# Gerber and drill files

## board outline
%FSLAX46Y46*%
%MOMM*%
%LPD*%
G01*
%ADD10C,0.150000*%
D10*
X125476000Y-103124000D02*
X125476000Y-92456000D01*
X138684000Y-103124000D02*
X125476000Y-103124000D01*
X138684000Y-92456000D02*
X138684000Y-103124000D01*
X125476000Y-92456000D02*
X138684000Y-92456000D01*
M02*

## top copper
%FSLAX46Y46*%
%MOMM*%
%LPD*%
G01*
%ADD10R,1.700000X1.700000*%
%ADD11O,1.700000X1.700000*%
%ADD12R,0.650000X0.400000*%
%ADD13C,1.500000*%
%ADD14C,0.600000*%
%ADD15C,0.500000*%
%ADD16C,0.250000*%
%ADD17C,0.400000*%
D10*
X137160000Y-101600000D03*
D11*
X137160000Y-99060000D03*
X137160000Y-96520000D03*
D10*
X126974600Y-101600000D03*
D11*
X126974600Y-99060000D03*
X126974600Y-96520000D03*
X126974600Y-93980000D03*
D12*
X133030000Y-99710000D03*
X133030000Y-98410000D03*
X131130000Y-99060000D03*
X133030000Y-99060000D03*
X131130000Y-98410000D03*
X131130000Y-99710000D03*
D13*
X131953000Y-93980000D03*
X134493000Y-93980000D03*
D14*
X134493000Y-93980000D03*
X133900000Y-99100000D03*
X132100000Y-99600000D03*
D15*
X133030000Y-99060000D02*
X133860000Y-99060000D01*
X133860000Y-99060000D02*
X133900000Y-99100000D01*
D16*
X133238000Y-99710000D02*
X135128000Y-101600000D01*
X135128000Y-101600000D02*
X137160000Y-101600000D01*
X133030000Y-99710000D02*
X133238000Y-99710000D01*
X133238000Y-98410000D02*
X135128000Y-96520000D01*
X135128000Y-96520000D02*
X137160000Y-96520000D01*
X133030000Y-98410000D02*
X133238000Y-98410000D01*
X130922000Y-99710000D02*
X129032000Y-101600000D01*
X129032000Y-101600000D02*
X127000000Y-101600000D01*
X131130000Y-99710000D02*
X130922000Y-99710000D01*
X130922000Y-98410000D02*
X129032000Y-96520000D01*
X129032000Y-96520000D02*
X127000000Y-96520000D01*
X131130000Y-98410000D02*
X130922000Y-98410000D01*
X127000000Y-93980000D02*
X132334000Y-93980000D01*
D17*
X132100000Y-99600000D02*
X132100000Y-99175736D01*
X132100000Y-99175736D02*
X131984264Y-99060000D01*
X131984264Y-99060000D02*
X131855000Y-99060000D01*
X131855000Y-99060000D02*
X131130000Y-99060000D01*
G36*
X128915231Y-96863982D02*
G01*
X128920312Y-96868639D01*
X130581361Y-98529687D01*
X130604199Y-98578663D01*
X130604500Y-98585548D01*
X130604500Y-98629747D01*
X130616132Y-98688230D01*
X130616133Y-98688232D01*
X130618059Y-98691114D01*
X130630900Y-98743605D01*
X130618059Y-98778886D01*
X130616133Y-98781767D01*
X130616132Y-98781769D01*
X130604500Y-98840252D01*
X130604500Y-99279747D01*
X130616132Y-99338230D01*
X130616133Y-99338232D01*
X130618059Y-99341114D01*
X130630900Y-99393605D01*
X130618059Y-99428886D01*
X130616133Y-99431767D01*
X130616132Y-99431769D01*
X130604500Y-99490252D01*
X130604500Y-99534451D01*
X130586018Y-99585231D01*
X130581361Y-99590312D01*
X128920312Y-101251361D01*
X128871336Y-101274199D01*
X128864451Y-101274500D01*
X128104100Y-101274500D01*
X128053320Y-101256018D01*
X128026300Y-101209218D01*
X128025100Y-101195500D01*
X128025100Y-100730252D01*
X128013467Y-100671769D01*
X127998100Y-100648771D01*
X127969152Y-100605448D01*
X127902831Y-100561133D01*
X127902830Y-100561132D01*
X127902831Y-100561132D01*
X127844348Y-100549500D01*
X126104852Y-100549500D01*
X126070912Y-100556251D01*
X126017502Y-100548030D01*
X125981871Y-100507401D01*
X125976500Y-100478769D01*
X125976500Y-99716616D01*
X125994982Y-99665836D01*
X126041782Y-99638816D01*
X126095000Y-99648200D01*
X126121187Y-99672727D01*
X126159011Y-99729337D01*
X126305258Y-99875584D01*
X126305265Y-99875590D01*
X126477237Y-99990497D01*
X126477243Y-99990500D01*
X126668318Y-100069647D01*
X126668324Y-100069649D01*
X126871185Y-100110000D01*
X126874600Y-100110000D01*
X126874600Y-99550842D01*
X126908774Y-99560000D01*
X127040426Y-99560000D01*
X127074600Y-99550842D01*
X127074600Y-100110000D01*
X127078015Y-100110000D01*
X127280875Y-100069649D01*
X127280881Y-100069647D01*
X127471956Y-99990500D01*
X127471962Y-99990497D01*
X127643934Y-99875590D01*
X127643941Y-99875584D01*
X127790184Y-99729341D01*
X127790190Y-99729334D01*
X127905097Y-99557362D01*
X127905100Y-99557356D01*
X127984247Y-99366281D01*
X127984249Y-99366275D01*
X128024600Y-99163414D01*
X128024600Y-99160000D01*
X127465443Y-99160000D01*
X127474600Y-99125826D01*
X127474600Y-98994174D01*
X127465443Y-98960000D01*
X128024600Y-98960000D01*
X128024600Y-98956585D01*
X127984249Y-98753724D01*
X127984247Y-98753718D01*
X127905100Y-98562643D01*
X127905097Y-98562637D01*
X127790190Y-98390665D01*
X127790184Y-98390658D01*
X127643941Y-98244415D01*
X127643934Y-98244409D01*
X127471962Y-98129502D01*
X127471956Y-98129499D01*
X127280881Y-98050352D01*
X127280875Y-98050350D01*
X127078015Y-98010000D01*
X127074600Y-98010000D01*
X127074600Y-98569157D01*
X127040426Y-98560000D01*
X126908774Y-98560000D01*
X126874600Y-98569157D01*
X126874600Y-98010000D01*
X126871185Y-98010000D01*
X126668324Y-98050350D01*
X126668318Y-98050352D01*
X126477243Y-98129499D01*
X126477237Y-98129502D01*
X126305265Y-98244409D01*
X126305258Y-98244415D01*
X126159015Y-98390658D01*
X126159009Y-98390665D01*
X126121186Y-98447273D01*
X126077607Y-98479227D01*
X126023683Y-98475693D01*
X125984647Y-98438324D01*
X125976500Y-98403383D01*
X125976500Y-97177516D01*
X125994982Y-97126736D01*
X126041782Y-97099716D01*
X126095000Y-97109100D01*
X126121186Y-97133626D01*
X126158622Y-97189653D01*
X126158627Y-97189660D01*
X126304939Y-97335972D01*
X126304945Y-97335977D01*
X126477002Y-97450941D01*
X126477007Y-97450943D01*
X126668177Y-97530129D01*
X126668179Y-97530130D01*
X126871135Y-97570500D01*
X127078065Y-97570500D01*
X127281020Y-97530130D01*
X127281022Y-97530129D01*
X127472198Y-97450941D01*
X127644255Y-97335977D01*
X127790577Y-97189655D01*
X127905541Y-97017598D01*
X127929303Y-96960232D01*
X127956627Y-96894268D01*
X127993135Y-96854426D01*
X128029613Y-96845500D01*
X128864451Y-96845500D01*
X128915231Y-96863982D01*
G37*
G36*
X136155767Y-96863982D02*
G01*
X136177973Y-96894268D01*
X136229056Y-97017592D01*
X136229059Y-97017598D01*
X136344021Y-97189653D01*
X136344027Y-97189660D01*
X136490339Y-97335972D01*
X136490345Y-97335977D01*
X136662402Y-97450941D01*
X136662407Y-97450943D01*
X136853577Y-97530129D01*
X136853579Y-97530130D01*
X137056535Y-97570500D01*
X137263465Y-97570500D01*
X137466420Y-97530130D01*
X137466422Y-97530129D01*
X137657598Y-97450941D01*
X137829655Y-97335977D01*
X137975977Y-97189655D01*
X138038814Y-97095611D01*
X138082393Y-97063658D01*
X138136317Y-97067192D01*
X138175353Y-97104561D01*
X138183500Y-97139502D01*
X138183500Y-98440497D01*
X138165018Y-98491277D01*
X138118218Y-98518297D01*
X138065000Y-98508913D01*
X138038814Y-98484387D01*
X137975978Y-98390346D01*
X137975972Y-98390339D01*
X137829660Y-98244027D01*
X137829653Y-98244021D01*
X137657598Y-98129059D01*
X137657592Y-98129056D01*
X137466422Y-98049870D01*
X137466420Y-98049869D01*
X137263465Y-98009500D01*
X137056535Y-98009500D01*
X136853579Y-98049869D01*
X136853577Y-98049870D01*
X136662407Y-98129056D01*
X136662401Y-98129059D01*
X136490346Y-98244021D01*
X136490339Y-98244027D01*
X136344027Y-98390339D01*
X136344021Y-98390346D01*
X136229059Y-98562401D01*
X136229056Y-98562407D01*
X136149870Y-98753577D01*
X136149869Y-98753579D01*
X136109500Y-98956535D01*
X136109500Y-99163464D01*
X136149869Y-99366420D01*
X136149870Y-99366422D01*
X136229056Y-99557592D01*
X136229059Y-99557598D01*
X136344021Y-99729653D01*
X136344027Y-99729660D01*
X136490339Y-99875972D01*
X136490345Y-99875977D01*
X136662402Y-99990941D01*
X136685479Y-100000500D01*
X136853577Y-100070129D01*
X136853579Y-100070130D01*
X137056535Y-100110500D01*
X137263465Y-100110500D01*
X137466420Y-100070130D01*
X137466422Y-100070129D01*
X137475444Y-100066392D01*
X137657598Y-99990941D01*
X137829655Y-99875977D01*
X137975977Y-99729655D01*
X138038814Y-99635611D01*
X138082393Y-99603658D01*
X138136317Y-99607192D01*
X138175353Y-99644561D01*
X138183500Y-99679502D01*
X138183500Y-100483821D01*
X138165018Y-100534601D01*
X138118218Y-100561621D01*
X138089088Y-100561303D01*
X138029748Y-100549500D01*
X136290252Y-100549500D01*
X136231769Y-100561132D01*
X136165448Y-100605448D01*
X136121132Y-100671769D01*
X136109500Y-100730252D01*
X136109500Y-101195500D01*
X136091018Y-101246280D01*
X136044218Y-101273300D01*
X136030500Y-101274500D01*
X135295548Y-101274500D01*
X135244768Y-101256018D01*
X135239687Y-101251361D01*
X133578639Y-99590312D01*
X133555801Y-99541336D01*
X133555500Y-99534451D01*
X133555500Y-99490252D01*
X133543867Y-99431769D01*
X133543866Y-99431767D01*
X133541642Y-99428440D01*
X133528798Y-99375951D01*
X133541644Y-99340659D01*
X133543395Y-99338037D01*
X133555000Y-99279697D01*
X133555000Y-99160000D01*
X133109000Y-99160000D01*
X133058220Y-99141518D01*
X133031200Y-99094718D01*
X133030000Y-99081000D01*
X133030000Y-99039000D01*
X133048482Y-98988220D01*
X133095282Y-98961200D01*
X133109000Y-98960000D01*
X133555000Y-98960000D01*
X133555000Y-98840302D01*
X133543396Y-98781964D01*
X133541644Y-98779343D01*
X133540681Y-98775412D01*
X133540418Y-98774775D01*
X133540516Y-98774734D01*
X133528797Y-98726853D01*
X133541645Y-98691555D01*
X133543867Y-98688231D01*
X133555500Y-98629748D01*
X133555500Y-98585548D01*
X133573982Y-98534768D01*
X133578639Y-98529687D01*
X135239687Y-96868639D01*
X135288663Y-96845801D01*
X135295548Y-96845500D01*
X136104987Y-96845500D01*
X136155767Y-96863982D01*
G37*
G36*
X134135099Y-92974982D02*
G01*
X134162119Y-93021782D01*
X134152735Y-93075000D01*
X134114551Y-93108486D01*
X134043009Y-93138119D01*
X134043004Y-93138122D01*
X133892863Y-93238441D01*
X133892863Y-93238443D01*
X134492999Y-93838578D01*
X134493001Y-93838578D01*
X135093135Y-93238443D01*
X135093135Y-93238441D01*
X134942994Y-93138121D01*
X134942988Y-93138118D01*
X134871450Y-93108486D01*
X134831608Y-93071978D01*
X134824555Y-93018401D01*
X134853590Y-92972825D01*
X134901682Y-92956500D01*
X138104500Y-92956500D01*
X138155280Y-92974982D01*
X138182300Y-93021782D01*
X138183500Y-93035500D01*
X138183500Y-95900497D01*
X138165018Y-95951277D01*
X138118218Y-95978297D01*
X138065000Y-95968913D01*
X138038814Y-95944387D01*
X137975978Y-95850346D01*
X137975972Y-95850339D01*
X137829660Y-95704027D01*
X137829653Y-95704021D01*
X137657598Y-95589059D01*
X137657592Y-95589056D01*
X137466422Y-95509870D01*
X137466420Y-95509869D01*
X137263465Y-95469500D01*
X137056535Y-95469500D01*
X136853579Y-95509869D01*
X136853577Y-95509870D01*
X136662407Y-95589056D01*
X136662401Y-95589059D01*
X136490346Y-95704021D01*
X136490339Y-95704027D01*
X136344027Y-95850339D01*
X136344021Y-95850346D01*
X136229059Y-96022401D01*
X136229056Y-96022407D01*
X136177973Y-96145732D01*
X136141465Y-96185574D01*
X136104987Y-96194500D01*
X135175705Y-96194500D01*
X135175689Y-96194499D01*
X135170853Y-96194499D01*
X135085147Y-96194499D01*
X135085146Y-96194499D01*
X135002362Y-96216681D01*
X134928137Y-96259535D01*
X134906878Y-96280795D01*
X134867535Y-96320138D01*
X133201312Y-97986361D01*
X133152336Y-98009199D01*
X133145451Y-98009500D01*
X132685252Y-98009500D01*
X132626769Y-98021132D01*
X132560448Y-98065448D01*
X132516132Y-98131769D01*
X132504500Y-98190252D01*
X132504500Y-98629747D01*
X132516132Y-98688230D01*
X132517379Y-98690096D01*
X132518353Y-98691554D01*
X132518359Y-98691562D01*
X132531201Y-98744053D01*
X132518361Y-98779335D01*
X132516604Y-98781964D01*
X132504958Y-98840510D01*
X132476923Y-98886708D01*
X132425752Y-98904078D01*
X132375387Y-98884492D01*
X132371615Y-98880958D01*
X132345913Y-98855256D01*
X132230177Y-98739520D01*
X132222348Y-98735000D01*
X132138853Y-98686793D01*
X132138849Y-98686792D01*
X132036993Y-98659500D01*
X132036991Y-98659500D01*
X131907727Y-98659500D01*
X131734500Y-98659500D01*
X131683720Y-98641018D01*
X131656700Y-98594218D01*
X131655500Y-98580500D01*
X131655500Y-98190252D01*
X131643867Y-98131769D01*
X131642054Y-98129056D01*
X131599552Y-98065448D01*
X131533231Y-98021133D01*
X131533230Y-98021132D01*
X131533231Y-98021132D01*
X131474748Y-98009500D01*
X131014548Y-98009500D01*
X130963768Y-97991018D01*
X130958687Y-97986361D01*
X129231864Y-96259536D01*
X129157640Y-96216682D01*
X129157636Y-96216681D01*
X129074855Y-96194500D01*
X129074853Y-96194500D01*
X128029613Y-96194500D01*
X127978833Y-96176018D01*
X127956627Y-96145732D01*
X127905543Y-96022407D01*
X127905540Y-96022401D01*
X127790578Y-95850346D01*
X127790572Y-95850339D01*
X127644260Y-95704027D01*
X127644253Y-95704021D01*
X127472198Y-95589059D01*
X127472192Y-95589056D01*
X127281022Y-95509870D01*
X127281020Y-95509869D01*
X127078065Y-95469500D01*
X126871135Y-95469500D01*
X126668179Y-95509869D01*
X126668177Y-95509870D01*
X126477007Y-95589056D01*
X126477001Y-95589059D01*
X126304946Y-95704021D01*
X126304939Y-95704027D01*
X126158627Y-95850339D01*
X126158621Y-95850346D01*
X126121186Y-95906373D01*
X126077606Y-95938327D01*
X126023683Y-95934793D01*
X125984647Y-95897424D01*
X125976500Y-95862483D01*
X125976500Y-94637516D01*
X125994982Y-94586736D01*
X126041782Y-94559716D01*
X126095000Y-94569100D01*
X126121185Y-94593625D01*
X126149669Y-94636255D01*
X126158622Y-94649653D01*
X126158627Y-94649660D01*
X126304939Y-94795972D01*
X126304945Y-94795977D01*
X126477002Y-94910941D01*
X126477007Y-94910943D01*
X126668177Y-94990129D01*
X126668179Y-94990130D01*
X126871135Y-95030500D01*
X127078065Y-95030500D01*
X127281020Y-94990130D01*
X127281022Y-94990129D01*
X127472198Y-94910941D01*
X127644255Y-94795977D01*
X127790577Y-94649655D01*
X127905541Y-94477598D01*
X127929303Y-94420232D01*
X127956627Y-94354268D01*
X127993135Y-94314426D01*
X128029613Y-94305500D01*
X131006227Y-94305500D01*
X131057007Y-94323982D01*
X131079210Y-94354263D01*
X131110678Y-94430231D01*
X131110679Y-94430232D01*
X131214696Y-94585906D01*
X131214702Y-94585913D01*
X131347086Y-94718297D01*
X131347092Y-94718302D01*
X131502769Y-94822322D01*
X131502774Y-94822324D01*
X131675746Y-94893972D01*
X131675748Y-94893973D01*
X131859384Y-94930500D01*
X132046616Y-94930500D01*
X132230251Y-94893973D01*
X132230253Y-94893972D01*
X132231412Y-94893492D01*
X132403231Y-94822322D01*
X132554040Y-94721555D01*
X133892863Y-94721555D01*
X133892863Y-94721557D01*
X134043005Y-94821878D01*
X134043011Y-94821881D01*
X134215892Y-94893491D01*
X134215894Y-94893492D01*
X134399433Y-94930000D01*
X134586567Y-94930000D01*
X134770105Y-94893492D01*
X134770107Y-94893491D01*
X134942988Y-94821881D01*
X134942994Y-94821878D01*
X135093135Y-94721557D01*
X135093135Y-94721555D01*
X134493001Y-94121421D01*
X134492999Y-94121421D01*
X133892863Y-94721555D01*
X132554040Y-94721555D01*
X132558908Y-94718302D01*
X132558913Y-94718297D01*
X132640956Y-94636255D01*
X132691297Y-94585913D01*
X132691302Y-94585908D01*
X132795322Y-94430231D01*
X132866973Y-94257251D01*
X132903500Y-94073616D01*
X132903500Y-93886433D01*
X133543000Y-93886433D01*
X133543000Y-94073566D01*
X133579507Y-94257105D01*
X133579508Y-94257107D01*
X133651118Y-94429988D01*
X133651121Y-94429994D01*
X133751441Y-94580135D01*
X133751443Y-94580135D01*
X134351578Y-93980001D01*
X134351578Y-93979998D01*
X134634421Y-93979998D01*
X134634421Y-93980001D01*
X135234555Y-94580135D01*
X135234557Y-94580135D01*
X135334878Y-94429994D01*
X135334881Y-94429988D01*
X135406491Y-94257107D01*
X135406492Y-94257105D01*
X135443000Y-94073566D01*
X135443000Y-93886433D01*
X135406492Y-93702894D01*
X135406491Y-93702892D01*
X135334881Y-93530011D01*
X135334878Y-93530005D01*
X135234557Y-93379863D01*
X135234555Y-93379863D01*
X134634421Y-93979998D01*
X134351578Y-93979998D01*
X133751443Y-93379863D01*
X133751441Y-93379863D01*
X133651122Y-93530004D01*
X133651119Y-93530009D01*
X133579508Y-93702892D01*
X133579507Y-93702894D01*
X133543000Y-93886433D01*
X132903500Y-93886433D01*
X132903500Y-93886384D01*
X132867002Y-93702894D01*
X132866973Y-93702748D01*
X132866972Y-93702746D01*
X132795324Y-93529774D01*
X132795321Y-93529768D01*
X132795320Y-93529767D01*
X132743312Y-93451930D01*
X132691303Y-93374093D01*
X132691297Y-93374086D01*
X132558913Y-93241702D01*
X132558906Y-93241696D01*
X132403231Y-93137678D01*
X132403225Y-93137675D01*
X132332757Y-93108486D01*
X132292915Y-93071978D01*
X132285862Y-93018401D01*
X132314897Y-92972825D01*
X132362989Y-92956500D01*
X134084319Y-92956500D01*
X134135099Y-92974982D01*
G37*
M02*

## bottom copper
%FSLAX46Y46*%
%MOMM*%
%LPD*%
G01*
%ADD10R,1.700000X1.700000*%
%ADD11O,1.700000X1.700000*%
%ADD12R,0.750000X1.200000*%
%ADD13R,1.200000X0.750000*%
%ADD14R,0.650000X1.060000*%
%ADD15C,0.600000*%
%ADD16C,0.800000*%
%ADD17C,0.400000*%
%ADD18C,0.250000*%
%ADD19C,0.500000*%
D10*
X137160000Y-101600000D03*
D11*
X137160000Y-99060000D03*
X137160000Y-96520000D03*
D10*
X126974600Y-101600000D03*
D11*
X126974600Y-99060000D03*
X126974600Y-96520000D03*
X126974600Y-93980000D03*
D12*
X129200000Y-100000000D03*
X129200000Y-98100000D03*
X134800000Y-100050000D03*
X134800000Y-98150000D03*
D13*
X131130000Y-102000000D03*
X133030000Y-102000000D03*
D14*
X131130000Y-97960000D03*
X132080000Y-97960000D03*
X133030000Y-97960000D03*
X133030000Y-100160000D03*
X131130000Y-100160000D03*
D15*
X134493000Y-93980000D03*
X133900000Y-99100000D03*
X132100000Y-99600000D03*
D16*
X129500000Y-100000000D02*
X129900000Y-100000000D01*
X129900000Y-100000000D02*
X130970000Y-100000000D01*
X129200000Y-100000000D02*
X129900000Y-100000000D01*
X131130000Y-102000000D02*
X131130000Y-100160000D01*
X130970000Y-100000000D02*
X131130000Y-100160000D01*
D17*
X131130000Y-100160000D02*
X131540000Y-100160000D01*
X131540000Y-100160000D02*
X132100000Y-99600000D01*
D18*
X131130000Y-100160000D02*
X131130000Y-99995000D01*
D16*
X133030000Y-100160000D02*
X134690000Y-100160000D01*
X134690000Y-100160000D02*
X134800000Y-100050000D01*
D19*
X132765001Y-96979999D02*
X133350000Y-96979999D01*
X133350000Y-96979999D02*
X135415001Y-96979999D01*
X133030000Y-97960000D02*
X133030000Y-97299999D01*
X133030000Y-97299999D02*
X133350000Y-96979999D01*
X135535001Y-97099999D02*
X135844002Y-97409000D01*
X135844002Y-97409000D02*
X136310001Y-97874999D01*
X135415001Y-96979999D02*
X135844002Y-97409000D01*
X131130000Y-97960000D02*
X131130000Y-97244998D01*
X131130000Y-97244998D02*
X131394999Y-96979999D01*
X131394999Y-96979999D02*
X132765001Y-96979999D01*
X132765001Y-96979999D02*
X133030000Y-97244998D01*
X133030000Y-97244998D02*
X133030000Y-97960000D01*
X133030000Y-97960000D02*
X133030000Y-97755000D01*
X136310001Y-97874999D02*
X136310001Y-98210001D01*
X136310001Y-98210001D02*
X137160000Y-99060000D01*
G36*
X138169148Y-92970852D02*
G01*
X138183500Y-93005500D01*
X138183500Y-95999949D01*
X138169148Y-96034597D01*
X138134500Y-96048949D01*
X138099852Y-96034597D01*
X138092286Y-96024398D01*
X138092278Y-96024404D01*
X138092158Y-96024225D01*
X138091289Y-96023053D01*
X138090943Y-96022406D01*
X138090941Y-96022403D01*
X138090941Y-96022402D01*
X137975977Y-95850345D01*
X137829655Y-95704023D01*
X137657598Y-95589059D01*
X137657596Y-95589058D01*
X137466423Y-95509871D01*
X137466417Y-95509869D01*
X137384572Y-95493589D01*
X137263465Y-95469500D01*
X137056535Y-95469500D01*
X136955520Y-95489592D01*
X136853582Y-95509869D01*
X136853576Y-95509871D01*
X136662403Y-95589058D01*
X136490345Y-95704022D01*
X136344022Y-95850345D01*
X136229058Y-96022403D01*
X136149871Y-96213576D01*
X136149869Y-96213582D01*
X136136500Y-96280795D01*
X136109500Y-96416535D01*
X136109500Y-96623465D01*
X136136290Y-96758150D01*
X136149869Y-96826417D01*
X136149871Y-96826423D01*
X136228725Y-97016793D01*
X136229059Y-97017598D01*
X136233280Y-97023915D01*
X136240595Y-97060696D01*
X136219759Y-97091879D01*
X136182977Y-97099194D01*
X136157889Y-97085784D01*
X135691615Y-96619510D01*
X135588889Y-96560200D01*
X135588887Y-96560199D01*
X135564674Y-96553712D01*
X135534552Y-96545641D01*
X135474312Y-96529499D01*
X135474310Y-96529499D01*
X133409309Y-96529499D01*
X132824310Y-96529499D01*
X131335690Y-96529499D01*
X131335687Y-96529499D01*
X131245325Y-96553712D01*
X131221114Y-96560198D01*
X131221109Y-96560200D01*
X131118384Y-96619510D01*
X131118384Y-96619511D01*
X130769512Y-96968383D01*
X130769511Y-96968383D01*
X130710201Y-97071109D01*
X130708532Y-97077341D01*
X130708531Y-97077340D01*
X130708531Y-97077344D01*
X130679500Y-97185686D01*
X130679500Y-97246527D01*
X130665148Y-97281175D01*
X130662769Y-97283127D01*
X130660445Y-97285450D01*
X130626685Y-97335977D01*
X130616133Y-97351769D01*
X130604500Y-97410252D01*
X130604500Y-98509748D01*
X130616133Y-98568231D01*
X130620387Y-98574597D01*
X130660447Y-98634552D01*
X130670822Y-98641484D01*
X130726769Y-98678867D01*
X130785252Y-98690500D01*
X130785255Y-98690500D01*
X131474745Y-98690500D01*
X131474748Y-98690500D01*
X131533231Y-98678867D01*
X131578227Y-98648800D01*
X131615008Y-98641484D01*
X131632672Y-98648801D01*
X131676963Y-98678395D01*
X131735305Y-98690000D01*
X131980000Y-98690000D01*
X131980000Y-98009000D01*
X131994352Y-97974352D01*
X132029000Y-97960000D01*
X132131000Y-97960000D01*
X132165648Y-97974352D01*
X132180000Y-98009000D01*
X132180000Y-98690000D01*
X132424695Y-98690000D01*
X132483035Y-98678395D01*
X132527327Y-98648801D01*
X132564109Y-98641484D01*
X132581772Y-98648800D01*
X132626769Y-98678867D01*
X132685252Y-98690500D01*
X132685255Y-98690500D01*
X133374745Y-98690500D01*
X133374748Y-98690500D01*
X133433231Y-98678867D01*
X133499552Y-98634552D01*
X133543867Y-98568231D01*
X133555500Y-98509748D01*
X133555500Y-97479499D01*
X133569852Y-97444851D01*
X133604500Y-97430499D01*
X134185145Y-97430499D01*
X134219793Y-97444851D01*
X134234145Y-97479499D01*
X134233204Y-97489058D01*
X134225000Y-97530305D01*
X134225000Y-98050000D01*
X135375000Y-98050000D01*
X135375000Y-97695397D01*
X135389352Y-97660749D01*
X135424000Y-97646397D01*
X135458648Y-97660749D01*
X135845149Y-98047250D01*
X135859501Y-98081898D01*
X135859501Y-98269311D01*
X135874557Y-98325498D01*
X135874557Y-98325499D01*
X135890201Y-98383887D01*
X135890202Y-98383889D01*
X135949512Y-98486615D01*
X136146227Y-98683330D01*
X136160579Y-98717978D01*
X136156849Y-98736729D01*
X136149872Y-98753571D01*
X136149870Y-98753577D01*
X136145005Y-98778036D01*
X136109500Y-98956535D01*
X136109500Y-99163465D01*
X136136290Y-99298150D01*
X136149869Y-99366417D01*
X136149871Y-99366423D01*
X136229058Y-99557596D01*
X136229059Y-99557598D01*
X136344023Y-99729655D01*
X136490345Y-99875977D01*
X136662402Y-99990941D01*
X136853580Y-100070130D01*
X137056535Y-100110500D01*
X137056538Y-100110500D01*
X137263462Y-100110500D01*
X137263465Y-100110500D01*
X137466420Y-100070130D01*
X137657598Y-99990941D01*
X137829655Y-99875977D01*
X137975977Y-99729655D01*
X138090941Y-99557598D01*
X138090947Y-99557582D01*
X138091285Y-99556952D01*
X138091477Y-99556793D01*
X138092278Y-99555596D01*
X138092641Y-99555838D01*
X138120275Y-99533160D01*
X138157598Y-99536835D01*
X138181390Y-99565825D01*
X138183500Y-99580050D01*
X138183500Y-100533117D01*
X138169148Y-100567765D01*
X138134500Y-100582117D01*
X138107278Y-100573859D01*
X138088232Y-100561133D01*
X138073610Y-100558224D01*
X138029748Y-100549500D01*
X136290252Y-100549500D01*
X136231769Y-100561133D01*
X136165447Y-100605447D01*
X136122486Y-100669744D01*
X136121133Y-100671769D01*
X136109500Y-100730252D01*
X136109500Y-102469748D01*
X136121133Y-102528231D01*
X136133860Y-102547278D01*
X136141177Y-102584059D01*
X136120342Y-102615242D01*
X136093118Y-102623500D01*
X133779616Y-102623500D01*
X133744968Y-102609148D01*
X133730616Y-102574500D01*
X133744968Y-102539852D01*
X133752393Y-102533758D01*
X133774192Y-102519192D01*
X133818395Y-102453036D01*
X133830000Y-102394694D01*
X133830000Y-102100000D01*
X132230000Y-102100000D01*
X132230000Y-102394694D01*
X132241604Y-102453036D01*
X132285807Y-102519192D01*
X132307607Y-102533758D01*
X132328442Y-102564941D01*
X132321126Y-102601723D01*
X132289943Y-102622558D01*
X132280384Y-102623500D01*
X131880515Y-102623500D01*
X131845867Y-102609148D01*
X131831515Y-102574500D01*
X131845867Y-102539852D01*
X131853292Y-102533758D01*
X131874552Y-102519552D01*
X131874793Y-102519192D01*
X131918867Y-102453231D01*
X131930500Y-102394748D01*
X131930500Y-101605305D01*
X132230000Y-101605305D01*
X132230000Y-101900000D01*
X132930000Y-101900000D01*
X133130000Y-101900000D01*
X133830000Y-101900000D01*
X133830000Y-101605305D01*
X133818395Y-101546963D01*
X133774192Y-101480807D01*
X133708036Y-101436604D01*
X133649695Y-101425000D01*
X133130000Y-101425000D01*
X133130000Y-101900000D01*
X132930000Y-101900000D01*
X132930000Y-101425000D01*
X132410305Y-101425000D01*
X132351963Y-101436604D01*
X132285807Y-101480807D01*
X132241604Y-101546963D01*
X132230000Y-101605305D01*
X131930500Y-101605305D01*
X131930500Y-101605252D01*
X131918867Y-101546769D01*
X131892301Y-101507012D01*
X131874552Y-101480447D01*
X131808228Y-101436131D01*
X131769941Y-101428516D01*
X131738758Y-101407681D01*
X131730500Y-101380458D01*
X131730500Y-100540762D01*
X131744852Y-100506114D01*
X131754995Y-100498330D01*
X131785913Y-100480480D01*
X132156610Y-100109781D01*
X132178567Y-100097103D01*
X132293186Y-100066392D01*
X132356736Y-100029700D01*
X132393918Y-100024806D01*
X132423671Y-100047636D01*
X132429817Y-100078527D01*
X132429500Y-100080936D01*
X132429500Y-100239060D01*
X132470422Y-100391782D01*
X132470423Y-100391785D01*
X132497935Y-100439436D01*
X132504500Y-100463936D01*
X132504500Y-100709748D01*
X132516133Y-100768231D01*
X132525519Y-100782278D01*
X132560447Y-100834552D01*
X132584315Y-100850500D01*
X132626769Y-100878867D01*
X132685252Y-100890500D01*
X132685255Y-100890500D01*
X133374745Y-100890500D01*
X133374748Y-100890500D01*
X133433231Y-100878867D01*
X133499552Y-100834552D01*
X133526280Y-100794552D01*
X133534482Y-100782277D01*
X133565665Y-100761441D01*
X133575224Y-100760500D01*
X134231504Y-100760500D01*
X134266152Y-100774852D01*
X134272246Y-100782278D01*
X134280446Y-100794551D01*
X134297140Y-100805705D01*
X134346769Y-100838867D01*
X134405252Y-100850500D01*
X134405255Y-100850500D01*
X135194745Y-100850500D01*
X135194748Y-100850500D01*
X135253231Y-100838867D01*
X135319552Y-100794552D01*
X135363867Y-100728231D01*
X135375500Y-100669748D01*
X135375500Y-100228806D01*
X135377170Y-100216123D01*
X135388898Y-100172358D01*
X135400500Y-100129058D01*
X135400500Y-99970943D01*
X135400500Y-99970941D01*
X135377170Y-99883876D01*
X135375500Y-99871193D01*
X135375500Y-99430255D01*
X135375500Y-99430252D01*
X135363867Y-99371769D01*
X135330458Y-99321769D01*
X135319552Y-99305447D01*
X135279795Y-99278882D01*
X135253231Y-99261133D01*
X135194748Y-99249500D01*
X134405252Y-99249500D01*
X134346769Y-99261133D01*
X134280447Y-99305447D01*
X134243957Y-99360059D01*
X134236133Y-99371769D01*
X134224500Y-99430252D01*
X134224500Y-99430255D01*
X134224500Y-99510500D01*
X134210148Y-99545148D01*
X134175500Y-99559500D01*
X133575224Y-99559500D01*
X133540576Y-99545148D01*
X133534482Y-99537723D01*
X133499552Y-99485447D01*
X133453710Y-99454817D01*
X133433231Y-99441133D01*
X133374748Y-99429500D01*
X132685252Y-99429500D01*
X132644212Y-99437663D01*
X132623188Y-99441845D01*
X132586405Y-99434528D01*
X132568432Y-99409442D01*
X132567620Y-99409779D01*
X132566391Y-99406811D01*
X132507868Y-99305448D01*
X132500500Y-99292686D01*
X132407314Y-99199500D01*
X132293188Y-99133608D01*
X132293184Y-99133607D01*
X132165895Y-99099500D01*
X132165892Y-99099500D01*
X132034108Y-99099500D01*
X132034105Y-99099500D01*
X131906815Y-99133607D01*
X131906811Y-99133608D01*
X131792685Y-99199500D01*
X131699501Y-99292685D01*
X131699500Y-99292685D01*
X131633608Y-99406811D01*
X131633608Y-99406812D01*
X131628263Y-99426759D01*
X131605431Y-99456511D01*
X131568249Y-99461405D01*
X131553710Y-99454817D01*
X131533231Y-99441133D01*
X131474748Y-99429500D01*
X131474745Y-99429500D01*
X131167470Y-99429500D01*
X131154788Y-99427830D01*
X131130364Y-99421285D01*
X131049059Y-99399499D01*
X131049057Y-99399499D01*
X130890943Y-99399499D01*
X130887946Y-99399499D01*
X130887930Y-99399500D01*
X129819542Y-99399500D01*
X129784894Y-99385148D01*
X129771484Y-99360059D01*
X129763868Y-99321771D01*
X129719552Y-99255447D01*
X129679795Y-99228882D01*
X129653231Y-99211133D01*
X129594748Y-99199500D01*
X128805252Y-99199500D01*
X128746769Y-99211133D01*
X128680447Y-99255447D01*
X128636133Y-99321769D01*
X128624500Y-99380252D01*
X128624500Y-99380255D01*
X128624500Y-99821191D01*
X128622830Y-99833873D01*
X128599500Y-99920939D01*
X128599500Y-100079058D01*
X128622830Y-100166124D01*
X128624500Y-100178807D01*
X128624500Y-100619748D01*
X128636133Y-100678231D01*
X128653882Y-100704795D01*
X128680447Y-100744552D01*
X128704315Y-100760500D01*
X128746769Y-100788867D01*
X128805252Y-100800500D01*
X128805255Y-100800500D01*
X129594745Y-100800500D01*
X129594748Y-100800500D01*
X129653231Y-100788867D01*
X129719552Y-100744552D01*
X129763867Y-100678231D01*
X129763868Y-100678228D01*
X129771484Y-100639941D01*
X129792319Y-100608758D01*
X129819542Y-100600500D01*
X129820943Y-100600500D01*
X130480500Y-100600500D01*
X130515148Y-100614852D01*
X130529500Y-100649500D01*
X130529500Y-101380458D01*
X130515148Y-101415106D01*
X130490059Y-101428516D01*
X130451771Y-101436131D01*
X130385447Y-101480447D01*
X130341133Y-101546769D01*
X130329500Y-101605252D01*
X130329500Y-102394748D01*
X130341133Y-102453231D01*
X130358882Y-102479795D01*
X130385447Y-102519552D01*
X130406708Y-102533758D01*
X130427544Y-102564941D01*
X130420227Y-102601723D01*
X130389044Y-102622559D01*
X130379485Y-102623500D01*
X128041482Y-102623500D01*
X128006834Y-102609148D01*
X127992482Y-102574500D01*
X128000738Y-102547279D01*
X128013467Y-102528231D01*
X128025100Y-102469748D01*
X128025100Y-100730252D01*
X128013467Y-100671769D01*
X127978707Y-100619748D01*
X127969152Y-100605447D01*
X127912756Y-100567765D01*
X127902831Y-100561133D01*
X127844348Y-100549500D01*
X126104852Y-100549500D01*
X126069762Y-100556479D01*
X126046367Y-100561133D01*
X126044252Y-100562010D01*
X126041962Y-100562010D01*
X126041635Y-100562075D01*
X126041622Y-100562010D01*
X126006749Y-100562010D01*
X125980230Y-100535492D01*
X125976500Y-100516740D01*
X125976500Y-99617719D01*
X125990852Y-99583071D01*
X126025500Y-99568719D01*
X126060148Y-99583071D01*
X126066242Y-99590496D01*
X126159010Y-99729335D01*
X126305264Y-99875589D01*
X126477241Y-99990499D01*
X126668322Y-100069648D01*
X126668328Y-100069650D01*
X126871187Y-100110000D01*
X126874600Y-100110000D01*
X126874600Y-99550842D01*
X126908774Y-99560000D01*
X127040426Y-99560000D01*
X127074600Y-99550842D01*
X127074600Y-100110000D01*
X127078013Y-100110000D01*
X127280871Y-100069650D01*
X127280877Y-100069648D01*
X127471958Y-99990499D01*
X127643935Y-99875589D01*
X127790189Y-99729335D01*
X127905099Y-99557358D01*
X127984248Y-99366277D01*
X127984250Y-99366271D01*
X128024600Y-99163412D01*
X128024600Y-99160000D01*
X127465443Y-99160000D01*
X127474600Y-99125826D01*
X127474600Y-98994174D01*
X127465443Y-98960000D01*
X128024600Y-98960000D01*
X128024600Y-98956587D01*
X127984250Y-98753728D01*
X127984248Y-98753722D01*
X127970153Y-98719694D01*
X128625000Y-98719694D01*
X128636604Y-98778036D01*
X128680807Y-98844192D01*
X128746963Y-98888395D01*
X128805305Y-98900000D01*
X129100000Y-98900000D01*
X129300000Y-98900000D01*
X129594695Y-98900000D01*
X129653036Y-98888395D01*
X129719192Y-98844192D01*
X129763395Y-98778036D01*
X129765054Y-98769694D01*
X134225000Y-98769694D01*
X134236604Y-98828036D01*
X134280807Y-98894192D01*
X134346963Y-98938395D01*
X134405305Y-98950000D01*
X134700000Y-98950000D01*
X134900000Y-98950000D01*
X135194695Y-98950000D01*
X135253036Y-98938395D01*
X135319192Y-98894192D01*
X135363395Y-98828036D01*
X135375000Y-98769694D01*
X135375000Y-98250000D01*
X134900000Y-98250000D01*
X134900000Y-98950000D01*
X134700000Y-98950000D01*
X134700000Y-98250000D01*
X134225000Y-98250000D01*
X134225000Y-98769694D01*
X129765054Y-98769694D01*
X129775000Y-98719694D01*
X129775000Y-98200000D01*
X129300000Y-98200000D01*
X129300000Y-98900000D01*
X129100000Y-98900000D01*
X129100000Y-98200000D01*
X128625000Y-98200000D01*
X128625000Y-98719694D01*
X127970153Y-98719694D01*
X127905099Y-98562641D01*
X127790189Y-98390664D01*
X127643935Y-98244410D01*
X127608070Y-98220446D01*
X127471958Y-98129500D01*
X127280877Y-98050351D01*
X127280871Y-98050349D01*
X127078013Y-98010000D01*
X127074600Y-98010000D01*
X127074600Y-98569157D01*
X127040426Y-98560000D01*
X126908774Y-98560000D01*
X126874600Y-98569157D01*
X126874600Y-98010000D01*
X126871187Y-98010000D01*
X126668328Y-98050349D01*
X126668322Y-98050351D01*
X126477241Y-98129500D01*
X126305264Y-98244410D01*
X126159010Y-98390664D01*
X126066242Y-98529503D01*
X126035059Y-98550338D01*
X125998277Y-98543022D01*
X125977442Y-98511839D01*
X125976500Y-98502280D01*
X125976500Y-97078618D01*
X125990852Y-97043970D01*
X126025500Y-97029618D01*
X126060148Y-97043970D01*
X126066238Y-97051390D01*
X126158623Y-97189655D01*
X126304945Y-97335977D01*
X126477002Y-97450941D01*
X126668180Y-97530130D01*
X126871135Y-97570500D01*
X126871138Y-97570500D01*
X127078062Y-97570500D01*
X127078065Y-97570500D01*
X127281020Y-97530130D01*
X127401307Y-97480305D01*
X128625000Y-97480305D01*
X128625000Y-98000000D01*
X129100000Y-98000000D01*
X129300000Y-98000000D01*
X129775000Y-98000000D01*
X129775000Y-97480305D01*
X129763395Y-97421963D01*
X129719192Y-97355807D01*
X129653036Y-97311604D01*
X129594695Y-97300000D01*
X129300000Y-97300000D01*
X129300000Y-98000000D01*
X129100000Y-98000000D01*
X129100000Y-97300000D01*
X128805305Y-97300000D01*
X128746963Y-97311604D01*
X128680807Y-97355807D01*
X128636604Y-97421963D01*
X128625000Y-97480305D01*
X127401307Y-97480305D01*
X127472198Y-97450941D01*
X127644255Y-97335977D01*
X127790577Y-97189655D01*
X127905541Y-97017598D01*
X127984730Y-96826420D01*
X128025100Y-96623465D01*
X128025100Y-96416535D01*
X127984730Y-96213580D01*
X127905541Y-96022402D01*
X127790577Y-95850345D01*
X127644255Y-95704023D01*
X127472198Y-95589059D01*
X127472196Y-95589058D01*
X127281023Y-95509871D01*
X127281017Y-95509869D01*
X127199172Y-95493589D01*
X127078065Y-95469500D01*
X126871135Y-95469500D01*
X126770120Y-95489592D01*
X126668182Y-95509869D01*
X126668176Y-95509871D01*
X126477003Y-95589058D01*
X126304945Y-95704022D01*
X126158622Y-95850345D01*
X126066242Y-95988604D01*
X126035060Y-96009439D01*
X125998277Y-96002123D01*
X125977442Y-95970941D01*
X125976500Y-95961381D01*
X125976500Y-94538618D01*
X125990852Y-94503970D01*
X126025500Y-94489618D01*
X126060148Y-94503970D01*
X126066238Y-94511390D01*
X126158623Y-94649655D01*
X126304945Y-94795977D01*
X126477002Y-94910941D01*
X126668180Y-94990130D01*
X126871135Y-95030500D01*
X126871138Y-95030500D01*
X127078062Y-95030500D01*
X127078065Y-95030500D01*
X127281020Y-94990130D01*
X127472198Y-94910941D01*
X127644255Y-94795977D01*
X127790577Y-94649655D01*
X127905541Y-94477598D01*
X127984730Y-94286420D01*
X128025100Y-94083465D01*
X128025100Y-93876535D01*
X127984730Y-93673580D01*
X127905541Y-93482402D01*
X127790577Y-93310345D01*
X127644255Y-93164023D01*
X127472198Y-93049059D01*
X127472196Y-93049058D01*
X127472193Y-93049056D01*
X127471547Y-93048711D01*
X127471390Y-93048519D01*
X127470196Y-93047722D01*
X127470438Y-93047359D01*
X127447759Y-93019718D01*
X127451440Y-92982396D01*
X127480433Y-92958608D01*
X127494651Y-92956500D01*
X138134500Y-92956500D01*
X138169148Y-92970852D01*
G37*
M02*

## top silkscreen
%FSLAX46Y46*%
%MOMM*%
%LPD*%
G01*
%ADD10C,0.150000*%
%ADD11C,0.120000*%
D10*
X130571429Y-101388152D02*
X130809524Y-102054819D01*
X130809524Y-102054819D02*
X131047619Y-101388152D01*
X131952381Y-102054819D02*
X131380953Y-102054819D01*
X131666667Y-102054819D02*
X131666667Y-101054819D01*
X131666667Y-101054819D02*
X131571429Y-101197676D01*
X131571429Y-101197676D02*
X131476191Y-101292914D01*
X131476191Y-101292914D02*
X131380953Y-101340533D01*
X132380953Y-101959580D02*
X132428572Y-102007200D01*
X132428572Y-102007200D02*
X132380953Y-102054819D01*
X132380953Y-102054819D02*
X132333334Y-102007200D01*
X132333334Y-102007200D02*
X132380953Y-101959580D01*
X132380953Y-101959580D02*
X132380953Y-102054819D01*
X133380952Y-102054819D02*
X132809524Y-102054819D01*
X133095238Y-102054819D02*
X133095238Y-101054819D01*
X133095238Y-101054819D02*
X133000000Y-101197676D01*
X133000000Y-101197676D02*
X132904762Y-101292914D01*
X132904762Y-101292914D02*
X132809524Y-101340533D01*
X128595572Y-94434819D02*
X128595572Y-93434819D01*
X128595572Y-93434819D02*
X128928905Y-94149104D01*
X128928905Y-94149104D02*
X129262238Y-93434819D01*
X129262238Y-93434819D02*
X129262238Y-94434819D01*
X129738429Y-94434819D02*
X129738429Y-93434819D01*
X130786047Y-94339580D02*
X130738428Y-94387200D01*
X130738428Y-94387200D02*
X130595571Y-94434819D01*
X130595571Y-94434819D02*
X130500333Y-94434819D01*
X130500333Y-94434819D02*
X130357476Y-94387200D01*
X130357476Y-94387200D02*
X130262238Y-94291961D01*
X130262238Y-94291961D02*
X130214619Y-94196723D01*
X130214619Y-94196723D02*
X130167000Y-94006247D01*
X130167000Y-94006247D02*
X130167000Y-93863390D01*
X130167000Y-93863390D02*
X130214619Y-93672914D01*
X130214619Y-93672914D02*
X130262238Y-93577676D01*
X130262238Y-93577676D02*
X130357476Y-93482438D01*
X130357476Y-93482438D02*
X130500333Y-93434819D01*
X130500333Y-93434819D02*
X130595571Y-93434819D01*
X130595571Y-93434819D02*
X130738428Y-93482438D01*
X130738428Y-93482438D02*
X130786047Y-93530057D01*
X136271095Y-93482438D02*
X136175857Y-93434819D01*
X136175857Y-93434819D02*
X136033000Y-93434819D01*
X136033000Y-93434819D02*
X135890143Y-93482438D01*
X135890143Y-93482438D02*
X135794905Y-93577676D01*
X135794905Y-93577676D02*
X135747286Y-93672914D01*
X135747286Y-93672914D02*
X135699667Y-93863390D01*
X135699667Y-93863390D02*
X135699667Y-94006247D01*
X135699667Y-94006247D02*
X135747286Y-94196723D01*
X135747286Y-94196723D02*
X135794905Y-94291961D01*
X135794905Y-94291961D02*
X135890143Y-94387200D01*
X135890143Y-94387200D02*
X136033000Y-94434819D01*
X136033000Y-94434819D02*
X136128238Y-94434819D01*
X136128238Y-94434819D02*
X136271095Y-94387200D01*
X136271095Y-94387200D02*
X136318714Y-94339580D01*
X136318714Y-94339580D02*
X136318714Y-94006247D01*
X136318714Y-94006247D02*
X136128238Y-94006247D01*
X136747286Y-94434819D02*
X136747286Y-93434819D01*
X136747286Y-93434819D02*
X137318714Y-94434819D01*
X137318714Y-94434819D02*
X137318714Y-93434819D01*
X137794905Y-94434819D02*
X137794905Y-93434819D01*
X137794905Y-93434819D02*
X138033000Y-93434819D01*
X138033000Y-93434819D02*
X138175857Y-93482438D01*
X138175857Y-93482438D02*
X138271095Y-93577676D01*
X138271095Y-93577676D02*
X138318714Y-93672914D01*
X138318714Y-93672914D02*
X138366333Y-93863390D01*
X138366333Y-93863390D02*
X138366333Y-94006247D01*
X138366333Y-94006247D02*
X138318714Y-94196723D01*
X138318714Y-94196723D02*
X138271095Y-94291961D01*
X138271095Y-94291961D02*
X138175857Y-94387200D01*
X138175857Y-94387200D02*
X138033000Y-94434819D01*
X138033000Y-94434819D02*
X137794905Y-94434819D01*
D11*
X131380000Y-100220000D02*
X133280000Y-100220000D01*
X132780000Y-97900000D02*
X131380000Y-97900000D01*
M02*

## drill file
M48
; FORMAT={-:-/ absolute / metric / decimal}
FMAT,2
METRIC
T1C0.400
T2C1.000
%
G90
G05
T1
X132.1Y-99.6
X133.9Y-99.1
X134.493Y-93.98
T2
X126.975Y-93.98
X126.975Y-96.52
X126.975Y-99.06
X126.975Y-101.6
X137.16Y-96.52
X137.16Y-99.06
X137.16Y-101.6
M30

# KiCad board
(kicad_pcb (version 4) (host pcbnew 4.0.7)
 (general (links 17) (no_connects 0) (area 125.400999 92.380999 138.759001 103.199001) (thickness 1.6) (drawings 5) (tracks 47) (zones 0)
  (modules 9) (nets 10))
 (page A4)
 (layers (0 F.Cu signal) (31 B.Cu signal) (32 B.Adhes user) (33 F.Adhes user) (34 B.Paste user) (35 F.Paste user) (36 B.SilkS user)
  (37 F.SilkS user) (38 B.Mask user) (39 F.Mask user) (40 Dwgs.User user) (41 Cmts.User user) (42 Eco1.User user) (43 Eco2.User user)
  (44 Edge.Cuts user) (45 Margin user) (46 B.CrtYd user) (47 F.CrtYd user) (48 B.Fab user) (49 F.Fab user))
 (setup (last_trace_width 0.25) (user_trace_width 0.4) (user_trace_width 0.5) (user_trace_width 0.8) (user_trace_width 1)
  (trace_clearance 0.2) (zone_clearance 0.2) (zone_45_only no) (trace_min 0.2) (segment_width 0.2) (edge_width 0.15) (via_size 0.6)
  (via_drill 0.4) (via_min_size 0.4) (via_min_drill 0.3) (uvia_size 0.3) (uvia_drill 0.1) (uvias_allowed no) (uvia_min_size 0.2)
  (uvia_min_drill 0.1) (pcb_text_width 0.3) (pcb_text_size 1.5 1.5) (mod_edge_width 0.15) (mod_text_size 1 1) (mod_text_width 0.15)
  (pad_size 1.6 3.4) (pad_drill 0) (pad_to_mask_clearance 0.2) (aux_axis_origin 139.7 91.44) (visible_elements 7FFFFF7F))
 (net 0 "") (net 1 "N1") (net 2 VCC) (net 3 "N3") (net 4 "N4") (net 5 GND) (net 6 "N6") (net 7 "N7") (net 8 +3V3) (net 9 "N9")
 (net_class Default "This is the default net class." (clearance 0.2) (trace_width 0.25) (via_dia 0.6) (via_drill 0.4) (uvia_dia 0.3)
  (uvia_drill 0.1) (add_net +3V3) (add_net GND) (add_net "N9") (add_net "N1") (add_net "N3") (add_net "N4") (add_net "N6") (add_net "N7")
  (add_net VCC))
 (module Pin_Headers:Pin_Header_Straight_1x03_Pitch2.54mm (layer B.Cu) (at 137.16 101.6)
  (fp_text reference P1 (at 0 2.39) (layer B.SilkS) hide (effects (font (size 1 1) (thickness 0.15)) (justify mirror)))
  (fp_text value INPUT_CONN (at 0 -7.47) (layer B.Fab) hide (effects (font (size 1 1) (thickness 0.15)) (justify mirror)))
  (pad 1 thru_hole rect (at 0 0) (size 1.7 1.7) (drill 1) (layers *.Cu *.Mask) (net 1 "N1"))
  (pad 2 thru_hole oval (at 0 -2.54) (size 1.7 1.7) (drill 1) (layers *.Cu *.Mask) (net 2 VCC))
  (pad 3 thru_hole oval (at 0 -5.08) (size 1.7 1.7) (drill 1) (layers *.Cu *.Mask) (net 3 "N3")))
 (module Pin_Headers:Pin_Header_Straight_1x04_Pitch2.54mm (layer B.Cu) (at 126.9746 101.6)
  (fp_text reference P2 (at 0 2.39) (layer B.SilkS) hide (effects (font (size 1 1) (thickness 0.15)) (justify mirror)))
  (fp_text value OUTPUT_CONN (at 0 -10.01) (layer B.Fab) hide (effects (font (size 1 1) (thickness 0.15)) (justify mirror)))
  (pad 1 thru_hole rect (at 0 0) (size 1.7 1.7) (drill 1) (layers *.Cu *.Mask) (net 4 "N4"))
  (pad 2 thru_hole oval (at 0 -2.54) (size 1.7 1.7) (drill 1) (layers *.Cu *.Mask) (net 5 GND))
  (pad 3 thru_hole oval (at 0 -5.08) (size 1.7 1.7) (drill 1) (layers *.Cu *.Mask) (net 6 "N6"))
  (pad 4 thru_hole oval (at 0 -7.62) (size 1.7 1.7) (drill 1) (layers *.Cu *.Mask) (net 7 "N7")))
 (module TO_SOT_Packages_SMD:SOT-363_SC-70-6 (layer F.Cu) (at 132.08 99.06 180)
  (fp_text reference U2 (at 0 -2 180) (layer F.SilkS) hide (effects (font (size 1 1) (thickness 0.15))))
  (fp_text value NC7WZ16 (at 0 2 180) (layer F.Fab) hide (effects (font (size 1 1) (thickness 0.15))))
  (fp_line (start 0.7 -1.16) (end -1.2 -1.16) (layer F.SilkS) (width 0.12))
  (fp_line (start -0.7 1.16) (end 0.7 1.16) (layer F.SilkS) (width 0.12))
  (pad 1 smd rect (at -0.95 -0.65 180) (size 0.65 0.4) (layers F.Cu F.Paste F.Mask) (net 1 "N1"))
  (pad 3 smd rect (at -0.95 0.65 180) (size 0.65 0.4) (layers F.Cu F.Paste F.Mask) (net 3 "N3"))
  (pad 5 smd rect (at 0.95 0 180) (size 0.65 0.4) (layers F.Cu F.Paste F.Mask) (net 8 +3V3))
  (pad 2 smd rect (at -0.95 0 180) (size 0.65 0.4) (layers F.Cu F.Paste F.Mask) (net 5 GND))
  (pad 4 smd rect (at 0.95 0.65 180) (size 0.65 0.4) (layers F.Cu F.Paste F.Mask) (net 6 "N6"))
  (pad 6 smd rect (at 0.95 -0.65 180) (size 0.65 0.4) (layers F.Cu F.Paste F.Mask) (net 4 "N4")))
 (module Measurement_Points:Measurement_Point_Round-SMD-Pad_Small (layer F.Cu) (at 131.953 93.98)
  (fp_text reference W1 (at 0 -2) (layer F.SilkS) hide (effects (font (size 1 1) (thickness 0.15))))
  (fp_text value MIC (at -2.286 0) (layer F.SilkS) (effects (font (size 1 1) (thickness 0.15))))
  (pad 1 smd circle (at 0 0) (size 1.5 1.5) (layers F.Cu F.Mask) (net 7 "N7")))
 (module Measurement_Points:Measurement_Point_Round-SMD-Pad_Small (layer F.Cu) (at 134.493 93.98)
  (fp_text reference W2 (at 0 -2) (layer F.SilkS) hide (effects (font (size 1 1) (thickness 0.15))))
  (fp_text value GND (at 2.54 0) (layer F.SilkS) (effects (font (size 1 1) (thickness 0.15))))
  (pad 1 smd circle (at 0 0) (size 1.5 1.5) (layers F.Cu F.Mask) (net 5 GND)))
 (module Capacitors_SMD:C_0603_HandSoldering (layer B.Cu) (at 129.2 99.05 90)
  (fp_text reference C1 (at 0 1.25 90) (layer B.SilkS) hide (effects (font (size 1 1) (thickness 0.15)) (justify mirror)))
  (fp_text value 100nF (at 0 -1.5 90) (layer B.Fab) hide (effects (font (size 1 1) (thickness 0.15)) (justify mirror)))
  (pad 1 smd rect (at -0.95 0 90) (size 1.2 0.75) (layers B.Cu B.Paste B.Mask) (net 8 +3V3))
  (pad 2 smd rect (at 0.95 0 90) (size 1.2 0.75) (layers B.Cu B.Paste B.Mask) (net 5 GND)))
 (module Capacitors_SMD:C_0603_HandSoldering (layer B.Cu) (at 134.8 99.1 90)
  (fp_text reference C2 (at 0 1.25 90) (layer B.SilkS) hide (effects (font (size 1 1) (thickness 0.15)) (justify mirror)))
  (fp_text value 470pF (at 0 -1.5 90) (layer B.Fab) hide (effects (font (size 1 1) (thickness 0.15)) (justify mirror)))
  (pad 1 smd rect (at -0.95 0 90) (size 1.2 0.75) (layers B.Cu B.Paste B.Mask) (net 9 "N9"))
  (pad 2 smd rect (at 0.95 0 90) (size 1.2 0.75) (layers B.Cu B.Paste B.Mask) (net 5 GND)))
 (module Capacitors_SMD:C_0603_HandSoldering (layer B.Cu) (at 132.08 102)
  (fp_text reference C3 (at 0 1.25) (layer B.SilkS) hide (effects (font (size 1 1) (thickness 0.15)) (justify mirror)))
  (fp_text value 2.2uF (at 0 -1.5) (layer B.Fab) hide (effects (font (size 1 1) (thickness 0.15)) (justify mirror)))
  (pad 1 smd rect (at -0.95 0) (size 1.2 0.75) (layers B.Cu B.Paste B.Mask) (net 8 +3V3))
  (pad 2 smd rect (at 0.95 0) (size 1.2 0.75) (layers B.Cu B.Paste B.Mask) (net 5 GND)))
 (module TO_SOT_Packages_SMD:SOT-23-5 (layer B.Cu) (at 132.08 99.06 270)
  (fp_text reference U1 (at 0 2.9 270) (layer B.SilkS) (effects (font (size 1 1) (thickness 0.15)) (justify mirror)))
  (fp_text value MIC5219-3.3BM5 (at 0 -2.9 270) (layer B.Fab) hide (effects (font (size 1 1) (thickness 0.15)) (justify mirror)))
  (pad 1 smd rect (at -1.1 0.95 270) (size 1.06 0.65) (layers B.Cu B.Paste B.Mask) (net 2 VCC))
  (pad 2 smd rect (at -1.1 0 270) (size 1.06 0.65) (layers B.Cu B.Paste B.Mask) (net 5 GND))
  (pad 3 smd rect (at -1.1 -0.95 270) (size 1.06 0.65) (layers B.Cu B.Paste B.Mask) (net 2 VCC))
  (pad 4 smd rect (at 1.1 -0.95 270) (size 1.06 0.65) (layers B.Cu B.Paste B.Mask) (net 9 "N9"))
  (pad 5 smd rect (at 1.1 0.95 270) (size 1.06 0.65) (layers B.Cu B.Paste B.Mask) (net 8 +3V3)))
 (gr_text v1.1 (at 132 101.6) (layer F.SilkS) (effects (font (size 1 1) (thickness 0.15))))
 (gr_line (start 125.476 103.124) (end 125.476 92.456) (layer Edge.Cuts) (width 0.15))
 (gr_line (start 138.684 103.124) (end 125.476 103.124) (layer Edge.Cuts) (width 0.15))
 (gr_line (start 138.684 92.456) (end 138.684 103.124) (layer Edge.Cuts) (width 0.15))
 (gr_line (start 125.476 92.456) (end 138.684 92.456) (layer Edge.Cuts) (width 0.15))
 (via (at 134.493 93.98) (size 0.6) (drill 0.4) (layers F.Cu B.Cu) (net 5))
 (segment (start 133.03 99.06) (end 133.86 99.06) (width 0.5) (layer F.Cu) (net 5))
 (segment (start 133.86 99.06) (end 133.9 99.1) (width 0.5) (layer F.Cu) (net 5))
 (via (at 133.9 99.1) (size 0.6) (drill 0.4) (layers F.Cu B.Cu) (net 5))
 (segment (start 133.238 99.71) (end 135.128 101.6) (width 0.25) (layer F.Cu) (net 1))
 (segment (start 135.128 101.6) (end 137.16 101.6) (width 0.25) (layer F.Cu) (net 1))
 (segment (start 133.03 99.71) (end 133.238 99.71) (width 0.25) (layer F.Cu) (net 1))
 (segment (start 133.238 98.41) (end 135.128 96.52) (width 0.25) (layer F.Cu) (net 3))
 (segment (start 135.128 96.52) (end 137.16 96.52) (width 0.25) (layer F.Cu) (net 3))
 (segment (start 133.03 98.41) (end 133.238 98.41) (width 0.25) (layer F.Cu) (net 3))
 (segment (start 130.922 99.71) (end 129.032 101.6) (width 0.25) (layer F.Cu) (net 4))
 (segment (start 129.032 101.6) (end 127 101.6) (width 0.25) (layer F.Cu) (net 4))
 (segment (start 131.13 99.71) (end 130.922 99.71) (width 0.25) (layer F.Cu) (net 4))
 (segment (start 130.922 98.41) (end 129.032 96.52) (width 0.25) (layer F.Cu) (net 6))
 (segment (start 129.032 96.52) (end 127 96.52) (width 0.25) (layer F.Cu) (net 6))
 (segment (start 131.13 98.41) (end 130.922 98.41) (width 0.25) (layer F.Cu) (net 6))
 (segment (start 127 93.98) (end 132.334 93.98) (width 0.25) (layer F.Cu) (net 7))
 (segment (start 129.5 100) (end 129.9 100) (width 0.8) (layer B.Cu) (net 8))
 (segment (start 129.9 100) (end 130.97 100) (width 0.8) (layer B.Cu) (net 8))
 (segment (start 129.2 100) (end 129.9 100) (width 0.8) (layer B.Cu) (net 8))
 (segment (start 131.13 102) (end 131.13 100.16) (width 0.8) (layer B.Cu) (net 8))
 (segment (start 130.97 100) (end 131.13 100.16) (width 0.8) (layer B.Cu) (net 8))
 (segment (start 132.1 99.6) (end 132.1 99.175736) (width 0.4) (layer F.Cu) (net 8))
 (segment (start 132.1 99.175736) (end 131.984264 99.06) (width 0.4) (layer F.Cu) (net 8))
 (segment (start 131.984264 99.06) (end 131.855 99.06) (width 0.4) (layer F.Cu) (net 8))
 (segment (start 131.855 99.06) (end 131.13 99.06) (width 0.4) (layer F.Cu) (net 8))
 (segment (start 131.13 100.16) (end 131.54 100.16) (width 0.4) (layer B.Cu) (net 8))
 (segment (start 131.54 100.16) (end 132.1 99.6) (width 0.4) (layer B.Cu) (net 8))
 (via (at 132.1 99.6) (size 0.6) (drill 0.4) (layers F.Cu B.Cu) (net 8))
 (segment (start 131.13 100.16) (end 131.13 99.995) (width 0.25) (layer B.Cu) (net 8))
 (segment (start 133.03 100.16) (end 134.69 100.16) (width 0.8) (layer B.Cu) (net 9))
 (segment (start 134.69 100.16) (end 134.8 100.05) (width 0.8) (layer B.Cu) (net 9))
 (segment (start 132.765001 96.979999) (end 133.35 96.979999) (width 0.5) (layer B.Cu) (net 2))
 (segment (start 133.35 96.979999) (end 135.415001 96.979999) (width 0.5) (layer B.Cu) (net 2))
 (segment (start 133.03 97.96) (end 133.03 97.299999) (width 0.5) (layer B.Cu) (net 2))
 (segment (start 133.03 97.299999) (end 133.35 96.979999) (width 0.5) (layer B.Cu) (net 2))
 (segment (start 135.535001 97.099999) (end 135.844002 97.409) (width 0.5) (layer B.Cu) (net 2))
 (segment (start 135.844002 97.409) (end 136.310001 97.874999) (width 0.5) (layer B.Cu) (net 2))
 (segment (start 135.415001 96.979999) (end 135.844002 97.409) (width 0.5) (layer B.Cu) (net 2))
 (segment (start 131.13 97.96) (end 131.13 97.244998) (width 0.5) (layer B.Cu) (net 2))
 (segment (start 131.13 97.244998) (end 131.394999 96.979999) (width 0.5) (layer B.Cu) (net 2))
 (segment (start 131.394999 96.979999) (end 132.765001 96.979999) (width 0.5) (layer B.Cu) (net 2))
 (segment (start 132.765001 96.979999) (end 133.03 97.244998) (width 0.5) (layer B.Cu) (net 2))
 (segment (start 133.03 97.244998) (end 133.03 97.96) (width 0.5) (layer B.Cu) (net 2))
 (segment (start 133.03 97.96) (end 133.03 97.755) (width 0.5) (layer B.Cu) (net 2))
 (segment (start 136.310001 97.874999) (end 136.310001 98.210001) (width 0.5) (layer B.Cu) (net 2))
 (segment (start 136.310001 98.210001) (end 137.16 99.06) (width 0.5) (layer B.Cu) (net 2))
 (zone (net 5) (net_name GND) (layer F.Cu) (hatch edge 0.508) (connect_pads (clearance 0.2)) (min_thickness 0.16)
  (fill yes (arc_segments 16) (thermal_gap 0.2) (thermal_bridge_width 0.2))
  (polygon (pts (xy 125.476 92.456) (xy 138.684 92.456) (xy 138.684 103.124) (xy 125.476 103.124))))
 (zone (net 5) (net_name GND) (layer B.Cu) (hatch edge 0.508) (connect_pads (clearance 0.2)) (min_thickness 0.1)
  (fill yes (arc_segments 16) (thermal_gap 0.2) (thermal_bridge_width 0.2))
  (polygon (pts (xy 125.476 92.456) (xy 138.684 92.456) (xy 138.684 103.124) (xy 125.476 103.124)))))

